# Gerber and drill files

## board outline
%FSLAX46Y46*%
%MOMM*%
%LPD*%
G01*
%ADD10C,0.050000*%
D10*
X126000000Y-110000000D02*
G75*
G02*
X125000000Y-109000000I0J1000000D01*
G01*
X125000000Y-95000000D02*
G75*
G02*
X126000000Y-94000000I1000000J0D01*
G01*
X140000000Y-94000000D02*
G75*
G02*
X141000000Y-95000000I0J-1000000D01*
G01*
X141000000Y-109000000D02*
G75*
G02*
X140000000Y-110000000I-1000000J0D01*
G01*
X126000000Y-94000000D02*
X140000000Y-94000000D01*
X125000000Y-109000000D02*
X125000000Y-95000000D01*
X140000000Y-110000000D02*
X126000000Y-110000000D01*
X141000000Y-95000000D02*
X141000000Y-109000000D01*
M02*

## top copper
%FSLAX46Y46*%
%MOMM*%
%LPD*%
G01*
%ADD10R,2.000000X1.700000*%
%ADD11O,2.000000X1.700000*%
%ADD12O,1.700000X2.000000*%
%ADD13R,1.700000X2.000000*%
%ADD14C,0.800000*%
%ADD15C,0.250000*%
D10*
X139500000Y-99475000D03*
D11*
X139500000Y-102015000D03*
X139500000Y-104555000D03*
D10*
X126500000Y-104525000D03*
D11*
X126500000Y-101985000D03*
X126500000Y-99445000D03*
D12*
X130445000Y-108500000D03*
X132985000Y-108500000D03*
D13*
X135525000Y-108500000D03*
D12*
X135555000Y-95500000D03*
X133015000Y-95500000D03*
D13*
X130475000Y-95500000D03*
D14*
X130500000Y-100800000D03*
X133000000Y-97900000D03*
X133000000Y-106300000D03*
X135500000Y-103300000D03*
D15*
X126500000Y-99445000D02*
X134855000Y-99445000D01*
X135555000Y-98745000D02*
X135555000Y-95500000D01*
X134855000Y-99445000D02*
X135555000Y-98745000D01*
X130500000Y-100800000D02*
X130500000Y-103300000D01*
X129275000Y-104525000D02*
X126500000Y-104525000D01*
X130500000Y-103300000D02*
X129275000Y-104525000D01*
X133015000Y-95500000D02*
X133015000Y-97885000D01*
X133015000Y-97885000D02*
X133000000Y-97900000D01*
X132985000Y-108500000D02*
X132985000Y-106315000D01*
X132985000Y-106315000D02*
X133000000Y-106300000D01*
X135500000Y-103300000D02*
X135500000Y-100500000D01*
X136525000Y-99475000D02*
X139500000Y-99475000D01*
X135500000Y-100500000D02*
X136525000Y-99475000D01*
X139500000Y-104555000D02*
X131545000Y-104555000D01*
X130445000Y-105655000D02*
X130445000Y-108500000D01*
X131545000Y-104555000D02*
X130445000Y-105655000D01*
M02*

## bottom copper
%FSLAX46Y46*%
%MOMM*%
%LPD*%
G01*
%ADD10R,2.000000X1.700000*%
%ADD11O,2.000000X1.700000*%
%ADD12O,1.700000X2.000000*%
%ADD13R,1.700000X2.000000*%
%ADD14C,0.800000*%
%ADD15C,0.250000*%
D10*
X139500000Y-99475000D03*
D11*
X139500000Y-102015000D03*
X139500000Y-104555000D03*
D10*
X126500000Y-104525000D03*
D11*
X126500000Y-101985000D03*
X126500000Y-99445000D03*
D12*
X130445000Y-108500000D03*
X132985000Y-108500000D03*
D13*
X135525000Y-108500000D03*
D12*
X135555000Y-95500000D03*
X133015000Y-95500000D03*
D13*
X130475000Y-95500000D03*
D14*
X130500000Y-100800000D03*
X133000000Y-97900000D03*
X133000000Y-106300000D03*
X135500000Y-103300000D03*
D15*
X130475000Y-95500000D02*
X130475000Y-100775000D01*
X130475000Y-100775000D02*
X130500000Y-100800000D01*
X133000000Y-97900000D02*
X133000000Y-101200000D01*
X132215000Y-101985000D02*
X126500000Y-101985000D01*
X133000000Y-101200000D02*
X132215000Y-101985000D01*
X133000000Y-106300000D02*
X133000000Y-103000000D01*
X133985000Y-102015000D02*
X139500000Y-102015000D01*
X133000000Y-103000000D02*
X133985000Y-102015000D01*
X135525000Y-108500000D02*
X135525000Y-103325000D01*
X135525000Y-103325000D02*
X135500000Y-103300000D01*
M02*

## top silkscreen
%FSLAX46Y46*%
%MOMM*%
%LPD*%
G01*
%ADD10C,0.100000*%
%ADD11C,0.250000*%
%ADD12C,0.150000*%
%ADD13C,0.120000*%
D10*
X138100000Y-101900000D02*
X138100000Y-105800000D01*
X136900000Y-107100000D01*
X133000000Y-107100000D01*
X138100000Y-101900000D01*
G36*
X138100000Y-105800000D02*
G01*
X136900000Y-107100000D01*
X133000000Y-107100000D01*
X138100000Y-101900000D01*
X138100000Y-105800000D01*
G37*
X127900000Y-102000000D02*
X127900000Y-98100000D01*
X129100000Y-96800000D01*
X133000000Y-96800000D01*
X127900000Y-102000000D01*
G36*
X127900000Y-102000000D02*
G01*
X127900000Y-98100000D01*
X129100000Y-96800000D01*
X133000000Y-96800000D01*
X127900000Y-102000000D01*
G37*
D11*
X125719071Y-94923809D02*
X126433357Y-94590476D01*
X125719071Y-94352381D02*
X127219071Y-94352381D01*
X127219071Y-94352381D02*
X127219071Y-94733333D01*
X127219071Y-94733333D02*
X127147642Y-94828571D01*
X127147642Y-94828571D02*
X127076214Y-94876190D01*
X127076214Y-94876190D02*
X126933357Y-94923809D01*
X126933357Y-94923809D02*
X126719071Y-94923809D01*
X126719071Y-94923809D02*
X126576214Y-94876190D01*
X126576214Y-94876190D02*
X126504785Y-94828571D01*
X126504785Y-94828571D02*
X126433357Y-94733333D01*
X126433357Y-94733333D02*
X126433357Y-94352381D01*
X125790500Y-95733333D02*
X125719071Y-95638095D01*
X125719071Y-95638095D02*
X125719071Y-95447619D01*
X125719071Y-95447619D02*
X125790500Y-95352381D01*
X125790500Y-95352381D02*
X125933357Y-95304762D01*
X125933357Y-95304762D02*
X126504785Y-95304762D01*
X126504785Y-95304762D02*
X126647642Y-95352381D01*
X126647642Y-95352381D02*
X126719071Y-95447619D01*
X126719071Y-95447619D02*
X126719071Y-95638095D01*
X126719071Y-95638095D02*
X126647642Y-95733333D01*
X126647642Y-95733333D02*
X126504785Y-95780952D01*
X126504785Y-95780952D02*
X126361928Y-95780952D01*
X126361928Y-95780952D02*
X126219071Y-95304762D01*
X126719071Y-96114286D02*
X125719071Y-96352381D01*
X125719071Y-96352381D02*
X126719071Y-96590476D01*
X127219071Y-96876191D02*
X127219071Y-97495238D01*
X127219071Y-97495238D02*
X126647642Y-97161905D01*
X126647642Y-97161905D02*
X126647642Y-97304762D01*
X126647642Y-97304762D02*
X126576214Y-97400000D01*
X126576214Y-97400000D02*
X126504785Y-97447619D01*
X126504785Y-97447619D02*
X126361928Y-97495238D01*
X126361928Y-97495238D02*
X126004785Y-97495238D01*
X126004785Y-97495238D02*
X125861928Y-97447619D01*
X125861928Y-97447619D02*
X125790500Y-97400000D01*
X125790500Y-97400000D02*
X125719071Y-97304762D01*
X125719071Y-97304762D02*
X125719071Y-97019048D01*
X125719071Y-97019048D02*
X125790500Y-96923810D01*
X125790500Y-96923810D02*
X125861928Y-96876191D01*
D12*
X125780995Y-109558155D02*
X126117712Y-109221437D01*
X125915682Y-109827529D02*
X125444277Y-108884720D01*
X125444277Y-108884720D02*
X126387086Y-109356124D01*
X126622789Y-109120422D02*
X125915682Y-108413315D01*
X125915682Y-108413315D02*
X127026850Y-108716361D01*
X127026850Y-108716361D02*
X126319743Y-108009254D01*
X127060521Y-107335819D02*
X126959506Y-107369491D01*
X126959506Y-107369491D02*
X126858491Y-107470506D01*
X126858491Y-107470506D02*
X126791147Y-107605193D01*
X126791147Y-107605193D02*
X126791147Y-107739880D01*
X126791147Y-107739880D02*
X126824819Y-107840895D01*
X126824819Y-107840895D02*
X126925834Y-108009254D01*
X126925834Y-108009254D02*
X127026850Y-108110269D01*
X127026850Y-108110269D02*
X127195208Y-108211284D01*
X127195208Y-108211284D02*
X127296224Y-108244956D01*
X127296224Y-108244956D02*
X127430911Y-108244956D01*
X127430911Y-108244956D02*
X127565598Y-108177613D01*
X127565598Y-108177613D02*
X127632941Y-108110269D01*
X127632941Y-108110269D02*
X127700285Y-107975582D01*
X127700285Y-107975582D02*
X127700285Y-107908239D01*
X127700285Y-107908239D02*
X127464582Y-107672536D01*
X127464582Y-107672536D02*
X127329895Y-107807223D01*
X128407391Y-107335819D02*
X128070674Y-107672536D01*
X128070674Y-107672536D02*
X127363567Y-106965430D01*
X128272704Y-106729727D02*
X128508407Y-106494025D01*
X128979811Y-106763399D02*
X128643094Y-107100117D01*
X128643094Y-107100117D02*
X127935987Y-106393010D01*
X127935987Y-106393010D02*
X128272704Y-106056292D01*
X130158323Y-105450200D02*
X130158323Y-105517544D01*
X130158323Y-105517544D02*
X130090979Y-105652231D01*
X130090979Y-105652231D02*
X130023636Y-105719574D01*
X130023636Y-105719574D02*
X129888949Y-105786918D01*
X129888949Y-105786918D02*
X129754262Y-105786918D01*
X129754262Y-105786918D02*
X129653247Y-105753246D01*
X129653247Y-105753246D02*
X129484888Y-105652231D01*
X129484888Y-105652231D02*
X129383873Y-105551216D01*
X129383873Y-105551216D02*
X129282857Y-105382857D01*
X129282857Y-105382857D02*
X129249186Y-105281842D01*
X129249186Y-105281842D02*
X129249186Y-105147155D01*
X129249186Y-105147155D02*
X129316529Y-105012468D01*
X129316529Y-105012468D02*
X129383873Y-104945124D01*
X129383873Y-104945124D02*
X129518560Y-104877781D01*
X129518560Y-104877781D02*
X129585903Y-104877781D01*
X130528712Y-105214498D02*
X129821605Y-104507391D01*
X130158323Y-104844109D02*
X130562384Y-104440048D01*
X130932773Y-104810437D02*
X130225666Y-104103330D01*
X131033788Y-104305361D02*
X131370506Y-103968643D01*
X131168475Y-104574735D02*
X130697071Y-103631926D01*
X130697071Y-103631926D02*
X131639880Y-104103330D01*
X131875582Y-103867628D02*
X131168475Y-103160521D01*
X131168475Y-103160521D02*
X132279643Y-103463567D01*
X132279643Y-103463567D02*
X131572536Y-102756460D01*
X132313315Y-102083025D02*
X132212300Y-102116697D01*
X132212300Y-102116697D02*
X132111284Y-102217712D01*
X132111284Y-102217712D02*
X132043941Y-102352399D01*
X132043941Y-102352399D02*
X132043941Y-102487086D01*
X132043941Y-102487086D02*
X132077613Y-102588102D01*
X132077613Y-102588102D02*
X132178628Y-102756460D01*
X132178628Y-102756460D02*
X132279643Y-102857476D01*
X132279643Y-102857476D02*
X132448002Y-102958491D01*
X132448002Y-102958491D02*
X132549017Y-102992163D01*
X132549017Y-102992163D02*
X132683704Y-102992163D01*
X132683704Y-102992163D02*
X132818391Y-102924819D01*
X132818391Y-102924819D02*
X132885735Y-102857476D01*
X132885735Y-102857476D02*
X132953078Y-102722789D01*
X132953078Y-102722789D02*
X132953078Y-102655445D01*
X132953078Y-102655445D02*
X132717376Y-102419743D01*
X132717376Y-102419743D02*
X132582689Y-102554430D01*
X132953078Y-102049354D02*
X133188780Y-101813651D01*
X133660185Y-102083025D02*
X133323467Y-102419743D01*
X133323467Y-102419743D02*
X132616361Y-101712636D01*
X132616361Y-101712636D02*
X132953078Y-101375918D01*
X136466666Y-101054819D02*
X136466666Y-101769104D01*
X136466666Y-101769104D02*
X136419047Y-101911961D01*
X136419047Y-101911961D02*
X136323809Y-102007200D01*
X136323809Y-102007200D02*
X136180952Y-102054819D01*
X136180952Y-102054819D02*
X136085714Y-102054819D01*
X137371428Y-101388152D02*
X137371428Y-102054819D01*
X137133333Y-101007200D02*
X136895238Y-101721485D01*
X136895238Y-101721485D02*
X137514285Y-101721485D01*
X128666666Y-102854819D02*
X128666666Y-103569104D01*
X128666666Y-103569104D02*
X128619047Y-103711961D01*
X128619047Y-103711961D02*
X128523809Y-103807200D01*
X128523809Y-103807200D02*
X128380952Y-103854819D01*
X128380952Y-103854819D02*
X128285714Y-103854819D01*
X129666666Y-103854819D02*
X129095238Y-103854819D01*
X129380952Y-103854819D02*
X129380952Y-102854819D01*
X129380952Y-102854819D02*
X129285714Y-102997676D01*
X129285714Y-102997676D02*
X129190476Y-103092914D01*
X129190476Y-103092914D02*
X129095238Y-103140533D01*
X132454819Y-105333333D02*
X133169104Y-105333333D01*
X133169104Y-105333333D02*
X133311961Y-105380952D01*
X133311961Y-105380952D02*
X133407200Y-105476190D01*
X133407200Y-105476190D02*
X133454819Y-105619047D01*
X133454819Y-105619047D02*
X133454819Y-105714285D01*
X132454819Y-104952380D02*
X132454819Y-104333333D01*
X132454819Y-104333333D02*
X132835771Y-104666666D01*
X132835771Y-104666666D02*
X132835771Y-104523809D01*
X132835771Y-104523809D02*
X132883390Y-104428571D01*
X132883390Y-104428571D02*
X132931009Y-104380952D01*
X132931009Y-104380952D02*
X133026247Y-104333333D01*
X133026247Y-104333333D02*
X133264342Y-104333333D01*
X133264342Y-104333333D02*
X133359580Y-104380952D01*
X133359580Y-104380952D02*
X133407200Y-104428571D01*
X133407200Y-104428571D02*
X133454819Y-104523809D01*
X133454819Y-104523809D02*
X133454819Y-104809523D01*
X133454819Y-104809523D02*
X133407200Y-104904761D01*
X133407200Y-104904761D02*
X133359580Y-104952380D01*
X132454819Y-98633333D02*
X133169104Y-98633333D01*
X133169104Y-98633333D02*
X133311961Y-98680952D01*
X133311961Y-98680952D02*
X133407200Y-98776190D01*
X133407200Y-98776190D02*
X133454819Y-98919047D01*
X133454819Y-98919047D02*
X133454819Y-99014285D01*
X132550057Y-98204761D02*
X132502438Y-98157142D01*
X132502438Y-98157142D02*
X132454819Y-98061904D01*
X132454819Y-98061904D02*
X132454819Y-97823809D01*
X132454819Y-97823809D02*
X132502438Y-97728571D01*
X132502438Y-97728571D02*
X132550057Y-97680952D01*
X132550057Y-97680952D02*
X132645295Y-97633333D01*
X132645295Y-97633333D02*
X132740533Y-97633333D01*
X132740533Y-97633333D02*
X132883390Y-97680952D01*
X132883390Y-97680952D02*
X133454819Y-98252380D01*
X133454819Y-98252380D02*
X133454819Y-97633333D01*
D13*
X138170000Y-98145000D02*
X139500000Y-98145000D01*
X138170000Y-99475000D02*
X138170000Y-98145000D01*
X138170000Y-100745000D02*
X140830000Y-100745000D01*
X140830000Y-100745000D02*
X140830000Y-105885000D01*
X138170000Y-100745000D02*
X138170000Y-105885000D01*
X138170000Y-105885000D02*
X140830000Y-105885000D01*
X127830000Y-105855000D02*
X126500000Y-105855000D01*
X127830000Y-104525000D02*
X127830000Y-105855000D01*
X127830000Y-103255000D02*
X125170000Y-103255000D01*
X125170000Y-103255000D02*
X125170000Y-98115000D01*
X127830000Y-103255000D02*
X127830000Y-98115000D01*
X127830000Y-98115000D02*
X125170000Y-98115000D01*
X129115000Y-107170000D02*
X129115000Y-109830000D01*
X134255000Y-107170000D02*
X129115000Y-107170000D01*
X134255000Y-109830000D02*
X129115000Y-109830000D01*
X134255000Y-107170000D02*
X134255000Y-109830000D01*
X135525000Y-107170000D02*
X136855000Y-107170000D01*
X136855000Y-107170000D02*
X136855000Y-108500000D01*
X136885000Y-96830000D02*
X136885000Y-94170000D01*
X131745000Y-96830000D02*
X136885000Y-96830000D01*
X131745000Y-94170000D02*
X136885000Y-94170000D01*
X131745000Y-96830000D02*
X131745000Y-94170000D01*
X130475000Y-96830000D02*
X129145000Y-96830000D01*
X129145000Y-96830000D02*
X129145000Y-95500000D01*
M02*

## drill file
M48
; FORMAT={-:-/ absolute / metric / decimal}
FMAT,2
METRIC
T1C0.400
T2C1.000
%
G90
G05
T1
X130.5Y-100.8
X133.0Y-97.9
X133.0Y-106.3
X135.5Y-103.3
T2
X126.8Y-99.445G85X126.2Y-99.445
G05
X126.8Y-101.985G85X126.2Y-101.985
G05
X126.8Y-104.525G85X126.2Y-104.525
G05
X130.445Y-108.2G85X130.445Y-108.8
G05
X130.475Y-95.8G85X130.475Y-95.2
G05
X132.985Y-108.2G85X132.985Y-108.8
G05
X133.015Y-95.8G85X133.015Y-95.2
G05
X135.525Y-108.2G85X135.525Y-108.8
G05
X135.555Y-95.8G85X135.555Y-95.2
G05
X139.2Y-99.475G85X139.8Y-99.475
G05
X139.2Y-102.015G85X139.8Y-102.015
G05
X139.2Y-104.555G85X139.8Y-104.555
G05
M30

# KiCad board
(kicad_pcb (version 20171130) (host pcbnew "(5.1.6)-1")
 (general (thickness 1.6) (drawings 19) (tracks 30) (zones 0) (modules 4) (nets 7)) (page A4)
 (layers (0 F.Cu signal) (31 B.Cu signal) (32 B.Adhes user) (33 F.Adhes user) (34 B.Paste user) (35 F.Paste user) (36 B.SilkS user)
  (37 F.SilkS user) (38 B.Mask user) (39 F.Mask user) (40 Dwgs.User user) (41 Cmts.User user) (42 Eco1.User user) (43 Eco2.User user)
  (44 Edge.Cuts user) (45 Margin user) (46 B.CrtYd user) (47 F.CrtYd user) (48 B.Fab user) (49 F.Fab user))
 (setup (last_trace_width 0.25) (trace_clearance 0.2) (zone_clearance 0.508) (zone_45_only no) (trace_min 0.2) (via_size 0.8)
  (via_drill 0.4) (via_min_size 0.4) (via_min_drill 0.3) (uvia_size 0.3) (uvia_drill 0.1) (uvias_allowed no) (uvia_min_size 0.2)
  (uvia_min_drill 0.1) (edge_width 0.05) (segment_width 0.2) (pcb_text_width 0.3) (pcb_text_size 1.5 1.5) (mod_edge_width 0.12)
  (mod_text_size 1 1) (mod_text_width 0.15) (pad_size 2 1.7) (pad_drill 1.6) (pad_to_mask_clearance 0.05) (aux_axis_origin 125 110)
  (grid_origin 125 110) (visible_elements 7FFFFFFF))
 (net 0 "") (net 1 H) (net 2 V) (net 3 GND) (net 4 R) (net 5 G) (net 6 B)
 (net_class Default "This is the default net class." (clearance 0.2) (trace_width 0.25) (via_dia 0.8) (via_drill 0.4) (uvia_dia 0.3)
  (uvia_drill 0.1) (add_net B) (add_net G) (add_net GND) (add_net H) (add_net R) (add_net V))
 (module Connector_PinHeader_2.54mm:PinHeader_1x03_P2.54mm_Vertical (layer F.Cu) (at 139.5 99.475)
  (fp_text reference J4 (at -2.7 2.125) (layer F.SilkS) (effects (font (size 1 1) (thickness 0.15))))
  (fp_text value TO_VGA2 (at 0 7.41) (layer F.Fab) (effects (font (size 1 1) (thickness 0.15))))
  (fp_line (start -1.33 -1.33) (end 0 -1.33) (layer F.SilkS) (width 0.12))
  (fp_line (start -1.33 0) (end -1.33 -1.33) (layer F.SilkS) (width 0.12))
  (fp_line (start -1.33 1.27) (end 1.33 1.27) (layer F.SilkS) (width 0.12))
  (fp_line (start 1.33 1.27) (end 1.33 6.41) (layer F.SilkS) (width 0.12))
  (fp_line (start -1.33 1.27) (end -1.33 6.41) (layer F.SilkS) (width 0.12))
  (fp_line (start -1.33 6.41) (end 1.33 6.41) (layer F.SilkS) (width 0.12))
  (pad 1 thru_hole rect (at 0 0) (size 2 1.7) (drill oval 1.6 1) (layers *.Cu *.Mask) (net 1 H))
  (pad 2 thru_hole oval (at 0 2.54) (size 2 1.7) (drill oval 1.6 1) (layers *.Cu *.Mask) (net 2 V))
  (pad 3 thru_hole oval (at 0 5.08) (size 2 1.7) (drill oval 1.6 1) (layers *.Cu *.Mask) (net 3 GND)))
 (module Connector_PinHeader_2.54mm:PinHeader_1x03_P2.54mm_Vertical (layer F.Cu) (at 126.5 104.525 180)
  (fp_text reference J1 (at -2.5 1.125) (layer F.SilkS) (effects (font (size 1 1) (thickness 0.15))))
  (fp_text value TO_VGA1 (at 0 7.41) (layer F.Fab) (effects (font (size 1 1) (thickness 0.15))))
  (fp_line (start -1.33 -1.33) (end 0 -1.33) (layer F.SilkS) (width 0.12))
  (fp_line (start -1.33 0) (end -1.33 -1.33) (layer F.SilkS) (width 0.12))
  (fp_line (start -1.33 1.27) (end 1.33 1.27) (layer F.SilkS) (width 0.12))
  (fp_line (start 1.33 1.27) (end 1.33 6.41) (layer F.SilkS) (width 0.12))
  (fp_line (start -1.33 1.27) (end -1.33 6.41) (layer F.SilkS) (width 0.12))
  (fp_line (start -1.33 6.41) (end 1.33 6.41) (layer F.SilkS) (width 0.12))
  (pad 1 thru_hole rect (at 0 0 180) (size 2 1.7) (drill oval 1.6 1) (layers *.Cu *.Mask) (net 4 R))
  (pad 2 thru_hole oval (at 0 2.54 180) (size 2 1.7) (drill oval 1.6 1) (layers *.Cu *.Mask) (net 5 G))
  (pad 3 thru_hole oval (at 0 5.08 180) (size 2 1.7) (drill oval 1.6 1) (layers *.Cu *.Mask) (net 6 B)))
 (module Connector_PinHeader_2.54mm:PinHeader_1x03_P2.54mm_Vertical (layer F.Cu) (at 135.525 108.5 270)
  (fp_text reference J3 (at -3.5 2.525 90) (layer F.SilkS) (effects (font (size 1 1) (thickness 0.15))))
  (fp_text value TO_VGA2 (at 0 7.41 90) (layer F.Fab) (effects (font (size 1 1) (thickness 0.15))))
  (fp_line (start -1.33 6.41) (end 1.33 6.41) (layer F.SilkS) (width 0.12))
  (fp_line (start -1.33 1.27) (end -1.33 6.41) (layer F.SilkS) (width 0.12))
  (fp_line (start 1.33 1.27) (end 1.33 6.41) (layer F.SilkS) (width 0.12))
  (fp_line (start -1.33 1.27) (end 1.33 1.27) (layer F.SilkS) (width 0.12))
  (fp_line (start -1.33 0) (end -1.33 -1.33) (layer F.SilkS) (width 0.12))
  (fp_line (start -1.33 -1.33) (end 0 -1.33) (layer F.SilkS) (width 0.12))
  (pad 3 thru_hole oval (at 0 5.08 270) (size 2 1.7) (drill oval 1.6 1) (layers *.Cu *.Mask) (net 3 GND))
  (pad 2 thru_hole oval (at 0 2.54 270) (size 2 1.7) (drill oval 1.6 1) (layers *.Cu *.Mask) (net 2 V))
  (pad 1 thru_hole rect (at 0 0 270) (size 2 1.7) (drill oval 1.6 1) (layers *.Cu *.Mask) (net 1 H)))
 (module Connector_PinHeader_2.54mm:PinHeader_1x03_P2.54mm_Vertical (layer F.Cu) (at 130.475 95.5 90)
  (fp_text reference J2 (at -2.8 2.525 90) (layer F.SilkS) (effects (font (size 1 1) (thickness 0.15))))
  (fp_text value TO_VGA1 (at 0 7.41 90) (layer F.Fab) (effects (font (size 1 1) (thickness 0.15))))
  (fp_line (start -1.33 6.41) (end 1.33 6.41) (layer F.SilkS) (width 0.12))
  (fp_line (start -1.33 1.27) (end -1.33 6.41) (layer F.SilkS) (width 0.12))
  (fp_line (start 1.33 1.27) (end 1.33 6.41) (layer F.SilkS) (width 0.12))
  (fp_line (start -1.33 1.27) (end 1.33 1.27) (layer F.SilkS) (width 0.12))
  (fp_line (start -1.33 0) (end -1.33 -1.33) (layer F.SilkS) (width 0.12))
  (fp_line (start -1.33 -1.33) (end 0 -1.33) (layer F.SilkS) (width 0.12))
  (pad 3 thru_hole oval (at 0 5.08 90) (size 2 1.7) (drill oval 1.6 1) (layers *.Cu *.Mask) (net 6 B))
  (pad 2 thru_hole oval (at 0 2.54 90) (size 2 1.7) (drill oval 1.6 1) (layers *.Cu *.Mask) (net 5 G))
  (pad 1 thru_hole rect (at 0 0 90) (size 2 1.7) (drill oval 1.6 1) (layers *.Cu *.Mask) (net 4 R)))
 (gr_poly (pts (xy 138.1 101.9) (xy 138.1 105.8) (xy 136.9 107.1) (xy 133 107.1)) (layer F.SilkS) (width 0.1))
 (gr_poly (pts (xy 127.9 102) (xy 127.9 98.1) (xy 129.1 96.8) (xy 133 96.8)) (layer F.SilkS) (width 0.1))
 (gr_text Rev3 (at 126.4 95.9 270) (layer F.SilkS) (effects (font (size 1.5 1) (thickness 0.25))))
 (gr_arc (start 126 109) (end 125 109) (angle -90) (layer Edge.Cuts) (width 0.05))
 (gr_arc (start 126 95) (end 126 94) (angle -90) (layer Edge.Cuts) (width 0.05))
 (gr_arc (start 140 95) (end 141 95) (angle -90) (layer Edge.Cuts) (width 0.05))
 (gr_arc (start 140 109) (end 140 110) (angle -90) (layer Edge.Cuts) (width 0.05))
 (gr_line (start 126 94) (end 140 94) (layer Edge.Cuts) (width 0.05))
 (gr_line (start 125 109) (end 125 95) (layer Edge.Cuts) (width 0.05))
 (gr_line (start 140 110) (end 126 110) (layer Edge.Cuts) (width 0.05))
 (gr_line (start 141 95) (end 141 109) (layer Edge.Cuts) (width 0.05))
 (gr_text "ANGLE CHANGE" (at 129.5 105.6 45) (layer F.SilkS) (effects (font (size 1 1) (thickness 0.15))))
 (segment (start 126.5 99.445) (end 134.855 99.445) (width 0.25) (layer F.Cu) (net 6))
 (segment (start 135.555 98.745) (end 135.555 95.5) (width 0.25) (layer F.Cu) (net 6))
 (segment (start 134.855 99.445) (end 135.555 98.745) (width 0.25) (layer F.Cu) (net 6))
 (via (at 130.5 100.8) (size 0.8) (drill 0.4) (layers F.Cu B.Cu) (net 4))
 (segment (start 130.475 95.5) (end 130.475 100.775) (width 0.25) (layer B.Cu) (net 4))
 (segment (start 130.475 100.775) (end 130.5 100.8) (width 0.25) (layer B.Cu) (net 4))
 (segment (start 130.5 100.8) (end 130.5 103.3) (width 0.25) (layer F.Cu) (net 4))
 (segment (start 129.275 104.525) (end 126.5 104.525) (width 0.25) (layer F.Cu) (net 4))
 (segment (start 130.5 103.3) (end 129.275 104.525) (width 0.25) (layer F.Cu) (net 4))
 (via (at 133 97.9) (size 0.8) (drill 0.4) (layers F.Cu B.Cu) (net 5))
 (segment (start 133.015 95.5) (end 133.015 97.885) (width 0.25) (layer F.Cu) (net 5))
 (segment (start 133.015 97.885) (end 133 97.9) (width 0.25) (layer F.Cu) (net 5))
 (segment (start 133 97.9) (end 133 101.2) (width 0.25) (layer B.Cu) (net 5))
 (segment (start 132.215 101.985) (end 126.5 101.985) (width 0.25) (layer B.Cu) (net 5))
 (segment (start 133 101.2) (end 132.215 101.985) (width 0.25) (layer B.Cu) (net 5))
 (via (at 133 106.3) (size 0.8) (drill 0.4) (layers F.Cu B.Cu) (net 2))
 (segment (start 132.985 108.5) (end 132.985 106.315) (width 0.25) (layer F.Cu) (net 2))
 (segment (start 132.985 106.315) (end 133 106.3) (width 0.25) (layer F.Cu) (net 2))
 (segment (start 133 106.3) (end 133 103) (width 0.25) (layer B.Cu) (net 2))
 (segment (start 133.985 102.015) (end 139.5 102.015) (width 0.25) (layer B.Cu) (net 2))
 (segment (start 133 103) (end 133.985 102.015) (width 0.25) (layer B.Cu) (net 2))
 (segment (start 135.525 108.5) (end 135.525 103.325) (width 0.25) (layer B.Cu) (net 1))
 (via (at 135.5 103.3) (size 0.8) (drill 0.4) (layers F.Cu B.Cu) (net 1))
 (segment (start 135.525 103.325) (end 135.5 103.3) (width 0.25) (layer B.Cu) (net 1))
 (segment (start 135.5 103.3) (end 135.5 100.5) (width 0.25) (layer F.Cu) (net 1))
 (segment (start 136.525 99.475) (end 139.5 99.475) (width 0.25) (layer F.Cu) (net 1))
 (segment (start 135.5 100.5) (end 136.525 99.475) (width 0.25) (layer F.Cu) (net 1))
 (segment (start 139.5 104.555) (end 131.545 104.555) (width 0.25) (layer F.Cu) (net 3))
 (segment (start 130.445 105.655) (end 130.445 108.5) (width 0.25) (layer F.Cu) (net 3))
 (segment (start 131.545 104.555) (end 130.445 105.655) (width 0.25) (layer F.Cu) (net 3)))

